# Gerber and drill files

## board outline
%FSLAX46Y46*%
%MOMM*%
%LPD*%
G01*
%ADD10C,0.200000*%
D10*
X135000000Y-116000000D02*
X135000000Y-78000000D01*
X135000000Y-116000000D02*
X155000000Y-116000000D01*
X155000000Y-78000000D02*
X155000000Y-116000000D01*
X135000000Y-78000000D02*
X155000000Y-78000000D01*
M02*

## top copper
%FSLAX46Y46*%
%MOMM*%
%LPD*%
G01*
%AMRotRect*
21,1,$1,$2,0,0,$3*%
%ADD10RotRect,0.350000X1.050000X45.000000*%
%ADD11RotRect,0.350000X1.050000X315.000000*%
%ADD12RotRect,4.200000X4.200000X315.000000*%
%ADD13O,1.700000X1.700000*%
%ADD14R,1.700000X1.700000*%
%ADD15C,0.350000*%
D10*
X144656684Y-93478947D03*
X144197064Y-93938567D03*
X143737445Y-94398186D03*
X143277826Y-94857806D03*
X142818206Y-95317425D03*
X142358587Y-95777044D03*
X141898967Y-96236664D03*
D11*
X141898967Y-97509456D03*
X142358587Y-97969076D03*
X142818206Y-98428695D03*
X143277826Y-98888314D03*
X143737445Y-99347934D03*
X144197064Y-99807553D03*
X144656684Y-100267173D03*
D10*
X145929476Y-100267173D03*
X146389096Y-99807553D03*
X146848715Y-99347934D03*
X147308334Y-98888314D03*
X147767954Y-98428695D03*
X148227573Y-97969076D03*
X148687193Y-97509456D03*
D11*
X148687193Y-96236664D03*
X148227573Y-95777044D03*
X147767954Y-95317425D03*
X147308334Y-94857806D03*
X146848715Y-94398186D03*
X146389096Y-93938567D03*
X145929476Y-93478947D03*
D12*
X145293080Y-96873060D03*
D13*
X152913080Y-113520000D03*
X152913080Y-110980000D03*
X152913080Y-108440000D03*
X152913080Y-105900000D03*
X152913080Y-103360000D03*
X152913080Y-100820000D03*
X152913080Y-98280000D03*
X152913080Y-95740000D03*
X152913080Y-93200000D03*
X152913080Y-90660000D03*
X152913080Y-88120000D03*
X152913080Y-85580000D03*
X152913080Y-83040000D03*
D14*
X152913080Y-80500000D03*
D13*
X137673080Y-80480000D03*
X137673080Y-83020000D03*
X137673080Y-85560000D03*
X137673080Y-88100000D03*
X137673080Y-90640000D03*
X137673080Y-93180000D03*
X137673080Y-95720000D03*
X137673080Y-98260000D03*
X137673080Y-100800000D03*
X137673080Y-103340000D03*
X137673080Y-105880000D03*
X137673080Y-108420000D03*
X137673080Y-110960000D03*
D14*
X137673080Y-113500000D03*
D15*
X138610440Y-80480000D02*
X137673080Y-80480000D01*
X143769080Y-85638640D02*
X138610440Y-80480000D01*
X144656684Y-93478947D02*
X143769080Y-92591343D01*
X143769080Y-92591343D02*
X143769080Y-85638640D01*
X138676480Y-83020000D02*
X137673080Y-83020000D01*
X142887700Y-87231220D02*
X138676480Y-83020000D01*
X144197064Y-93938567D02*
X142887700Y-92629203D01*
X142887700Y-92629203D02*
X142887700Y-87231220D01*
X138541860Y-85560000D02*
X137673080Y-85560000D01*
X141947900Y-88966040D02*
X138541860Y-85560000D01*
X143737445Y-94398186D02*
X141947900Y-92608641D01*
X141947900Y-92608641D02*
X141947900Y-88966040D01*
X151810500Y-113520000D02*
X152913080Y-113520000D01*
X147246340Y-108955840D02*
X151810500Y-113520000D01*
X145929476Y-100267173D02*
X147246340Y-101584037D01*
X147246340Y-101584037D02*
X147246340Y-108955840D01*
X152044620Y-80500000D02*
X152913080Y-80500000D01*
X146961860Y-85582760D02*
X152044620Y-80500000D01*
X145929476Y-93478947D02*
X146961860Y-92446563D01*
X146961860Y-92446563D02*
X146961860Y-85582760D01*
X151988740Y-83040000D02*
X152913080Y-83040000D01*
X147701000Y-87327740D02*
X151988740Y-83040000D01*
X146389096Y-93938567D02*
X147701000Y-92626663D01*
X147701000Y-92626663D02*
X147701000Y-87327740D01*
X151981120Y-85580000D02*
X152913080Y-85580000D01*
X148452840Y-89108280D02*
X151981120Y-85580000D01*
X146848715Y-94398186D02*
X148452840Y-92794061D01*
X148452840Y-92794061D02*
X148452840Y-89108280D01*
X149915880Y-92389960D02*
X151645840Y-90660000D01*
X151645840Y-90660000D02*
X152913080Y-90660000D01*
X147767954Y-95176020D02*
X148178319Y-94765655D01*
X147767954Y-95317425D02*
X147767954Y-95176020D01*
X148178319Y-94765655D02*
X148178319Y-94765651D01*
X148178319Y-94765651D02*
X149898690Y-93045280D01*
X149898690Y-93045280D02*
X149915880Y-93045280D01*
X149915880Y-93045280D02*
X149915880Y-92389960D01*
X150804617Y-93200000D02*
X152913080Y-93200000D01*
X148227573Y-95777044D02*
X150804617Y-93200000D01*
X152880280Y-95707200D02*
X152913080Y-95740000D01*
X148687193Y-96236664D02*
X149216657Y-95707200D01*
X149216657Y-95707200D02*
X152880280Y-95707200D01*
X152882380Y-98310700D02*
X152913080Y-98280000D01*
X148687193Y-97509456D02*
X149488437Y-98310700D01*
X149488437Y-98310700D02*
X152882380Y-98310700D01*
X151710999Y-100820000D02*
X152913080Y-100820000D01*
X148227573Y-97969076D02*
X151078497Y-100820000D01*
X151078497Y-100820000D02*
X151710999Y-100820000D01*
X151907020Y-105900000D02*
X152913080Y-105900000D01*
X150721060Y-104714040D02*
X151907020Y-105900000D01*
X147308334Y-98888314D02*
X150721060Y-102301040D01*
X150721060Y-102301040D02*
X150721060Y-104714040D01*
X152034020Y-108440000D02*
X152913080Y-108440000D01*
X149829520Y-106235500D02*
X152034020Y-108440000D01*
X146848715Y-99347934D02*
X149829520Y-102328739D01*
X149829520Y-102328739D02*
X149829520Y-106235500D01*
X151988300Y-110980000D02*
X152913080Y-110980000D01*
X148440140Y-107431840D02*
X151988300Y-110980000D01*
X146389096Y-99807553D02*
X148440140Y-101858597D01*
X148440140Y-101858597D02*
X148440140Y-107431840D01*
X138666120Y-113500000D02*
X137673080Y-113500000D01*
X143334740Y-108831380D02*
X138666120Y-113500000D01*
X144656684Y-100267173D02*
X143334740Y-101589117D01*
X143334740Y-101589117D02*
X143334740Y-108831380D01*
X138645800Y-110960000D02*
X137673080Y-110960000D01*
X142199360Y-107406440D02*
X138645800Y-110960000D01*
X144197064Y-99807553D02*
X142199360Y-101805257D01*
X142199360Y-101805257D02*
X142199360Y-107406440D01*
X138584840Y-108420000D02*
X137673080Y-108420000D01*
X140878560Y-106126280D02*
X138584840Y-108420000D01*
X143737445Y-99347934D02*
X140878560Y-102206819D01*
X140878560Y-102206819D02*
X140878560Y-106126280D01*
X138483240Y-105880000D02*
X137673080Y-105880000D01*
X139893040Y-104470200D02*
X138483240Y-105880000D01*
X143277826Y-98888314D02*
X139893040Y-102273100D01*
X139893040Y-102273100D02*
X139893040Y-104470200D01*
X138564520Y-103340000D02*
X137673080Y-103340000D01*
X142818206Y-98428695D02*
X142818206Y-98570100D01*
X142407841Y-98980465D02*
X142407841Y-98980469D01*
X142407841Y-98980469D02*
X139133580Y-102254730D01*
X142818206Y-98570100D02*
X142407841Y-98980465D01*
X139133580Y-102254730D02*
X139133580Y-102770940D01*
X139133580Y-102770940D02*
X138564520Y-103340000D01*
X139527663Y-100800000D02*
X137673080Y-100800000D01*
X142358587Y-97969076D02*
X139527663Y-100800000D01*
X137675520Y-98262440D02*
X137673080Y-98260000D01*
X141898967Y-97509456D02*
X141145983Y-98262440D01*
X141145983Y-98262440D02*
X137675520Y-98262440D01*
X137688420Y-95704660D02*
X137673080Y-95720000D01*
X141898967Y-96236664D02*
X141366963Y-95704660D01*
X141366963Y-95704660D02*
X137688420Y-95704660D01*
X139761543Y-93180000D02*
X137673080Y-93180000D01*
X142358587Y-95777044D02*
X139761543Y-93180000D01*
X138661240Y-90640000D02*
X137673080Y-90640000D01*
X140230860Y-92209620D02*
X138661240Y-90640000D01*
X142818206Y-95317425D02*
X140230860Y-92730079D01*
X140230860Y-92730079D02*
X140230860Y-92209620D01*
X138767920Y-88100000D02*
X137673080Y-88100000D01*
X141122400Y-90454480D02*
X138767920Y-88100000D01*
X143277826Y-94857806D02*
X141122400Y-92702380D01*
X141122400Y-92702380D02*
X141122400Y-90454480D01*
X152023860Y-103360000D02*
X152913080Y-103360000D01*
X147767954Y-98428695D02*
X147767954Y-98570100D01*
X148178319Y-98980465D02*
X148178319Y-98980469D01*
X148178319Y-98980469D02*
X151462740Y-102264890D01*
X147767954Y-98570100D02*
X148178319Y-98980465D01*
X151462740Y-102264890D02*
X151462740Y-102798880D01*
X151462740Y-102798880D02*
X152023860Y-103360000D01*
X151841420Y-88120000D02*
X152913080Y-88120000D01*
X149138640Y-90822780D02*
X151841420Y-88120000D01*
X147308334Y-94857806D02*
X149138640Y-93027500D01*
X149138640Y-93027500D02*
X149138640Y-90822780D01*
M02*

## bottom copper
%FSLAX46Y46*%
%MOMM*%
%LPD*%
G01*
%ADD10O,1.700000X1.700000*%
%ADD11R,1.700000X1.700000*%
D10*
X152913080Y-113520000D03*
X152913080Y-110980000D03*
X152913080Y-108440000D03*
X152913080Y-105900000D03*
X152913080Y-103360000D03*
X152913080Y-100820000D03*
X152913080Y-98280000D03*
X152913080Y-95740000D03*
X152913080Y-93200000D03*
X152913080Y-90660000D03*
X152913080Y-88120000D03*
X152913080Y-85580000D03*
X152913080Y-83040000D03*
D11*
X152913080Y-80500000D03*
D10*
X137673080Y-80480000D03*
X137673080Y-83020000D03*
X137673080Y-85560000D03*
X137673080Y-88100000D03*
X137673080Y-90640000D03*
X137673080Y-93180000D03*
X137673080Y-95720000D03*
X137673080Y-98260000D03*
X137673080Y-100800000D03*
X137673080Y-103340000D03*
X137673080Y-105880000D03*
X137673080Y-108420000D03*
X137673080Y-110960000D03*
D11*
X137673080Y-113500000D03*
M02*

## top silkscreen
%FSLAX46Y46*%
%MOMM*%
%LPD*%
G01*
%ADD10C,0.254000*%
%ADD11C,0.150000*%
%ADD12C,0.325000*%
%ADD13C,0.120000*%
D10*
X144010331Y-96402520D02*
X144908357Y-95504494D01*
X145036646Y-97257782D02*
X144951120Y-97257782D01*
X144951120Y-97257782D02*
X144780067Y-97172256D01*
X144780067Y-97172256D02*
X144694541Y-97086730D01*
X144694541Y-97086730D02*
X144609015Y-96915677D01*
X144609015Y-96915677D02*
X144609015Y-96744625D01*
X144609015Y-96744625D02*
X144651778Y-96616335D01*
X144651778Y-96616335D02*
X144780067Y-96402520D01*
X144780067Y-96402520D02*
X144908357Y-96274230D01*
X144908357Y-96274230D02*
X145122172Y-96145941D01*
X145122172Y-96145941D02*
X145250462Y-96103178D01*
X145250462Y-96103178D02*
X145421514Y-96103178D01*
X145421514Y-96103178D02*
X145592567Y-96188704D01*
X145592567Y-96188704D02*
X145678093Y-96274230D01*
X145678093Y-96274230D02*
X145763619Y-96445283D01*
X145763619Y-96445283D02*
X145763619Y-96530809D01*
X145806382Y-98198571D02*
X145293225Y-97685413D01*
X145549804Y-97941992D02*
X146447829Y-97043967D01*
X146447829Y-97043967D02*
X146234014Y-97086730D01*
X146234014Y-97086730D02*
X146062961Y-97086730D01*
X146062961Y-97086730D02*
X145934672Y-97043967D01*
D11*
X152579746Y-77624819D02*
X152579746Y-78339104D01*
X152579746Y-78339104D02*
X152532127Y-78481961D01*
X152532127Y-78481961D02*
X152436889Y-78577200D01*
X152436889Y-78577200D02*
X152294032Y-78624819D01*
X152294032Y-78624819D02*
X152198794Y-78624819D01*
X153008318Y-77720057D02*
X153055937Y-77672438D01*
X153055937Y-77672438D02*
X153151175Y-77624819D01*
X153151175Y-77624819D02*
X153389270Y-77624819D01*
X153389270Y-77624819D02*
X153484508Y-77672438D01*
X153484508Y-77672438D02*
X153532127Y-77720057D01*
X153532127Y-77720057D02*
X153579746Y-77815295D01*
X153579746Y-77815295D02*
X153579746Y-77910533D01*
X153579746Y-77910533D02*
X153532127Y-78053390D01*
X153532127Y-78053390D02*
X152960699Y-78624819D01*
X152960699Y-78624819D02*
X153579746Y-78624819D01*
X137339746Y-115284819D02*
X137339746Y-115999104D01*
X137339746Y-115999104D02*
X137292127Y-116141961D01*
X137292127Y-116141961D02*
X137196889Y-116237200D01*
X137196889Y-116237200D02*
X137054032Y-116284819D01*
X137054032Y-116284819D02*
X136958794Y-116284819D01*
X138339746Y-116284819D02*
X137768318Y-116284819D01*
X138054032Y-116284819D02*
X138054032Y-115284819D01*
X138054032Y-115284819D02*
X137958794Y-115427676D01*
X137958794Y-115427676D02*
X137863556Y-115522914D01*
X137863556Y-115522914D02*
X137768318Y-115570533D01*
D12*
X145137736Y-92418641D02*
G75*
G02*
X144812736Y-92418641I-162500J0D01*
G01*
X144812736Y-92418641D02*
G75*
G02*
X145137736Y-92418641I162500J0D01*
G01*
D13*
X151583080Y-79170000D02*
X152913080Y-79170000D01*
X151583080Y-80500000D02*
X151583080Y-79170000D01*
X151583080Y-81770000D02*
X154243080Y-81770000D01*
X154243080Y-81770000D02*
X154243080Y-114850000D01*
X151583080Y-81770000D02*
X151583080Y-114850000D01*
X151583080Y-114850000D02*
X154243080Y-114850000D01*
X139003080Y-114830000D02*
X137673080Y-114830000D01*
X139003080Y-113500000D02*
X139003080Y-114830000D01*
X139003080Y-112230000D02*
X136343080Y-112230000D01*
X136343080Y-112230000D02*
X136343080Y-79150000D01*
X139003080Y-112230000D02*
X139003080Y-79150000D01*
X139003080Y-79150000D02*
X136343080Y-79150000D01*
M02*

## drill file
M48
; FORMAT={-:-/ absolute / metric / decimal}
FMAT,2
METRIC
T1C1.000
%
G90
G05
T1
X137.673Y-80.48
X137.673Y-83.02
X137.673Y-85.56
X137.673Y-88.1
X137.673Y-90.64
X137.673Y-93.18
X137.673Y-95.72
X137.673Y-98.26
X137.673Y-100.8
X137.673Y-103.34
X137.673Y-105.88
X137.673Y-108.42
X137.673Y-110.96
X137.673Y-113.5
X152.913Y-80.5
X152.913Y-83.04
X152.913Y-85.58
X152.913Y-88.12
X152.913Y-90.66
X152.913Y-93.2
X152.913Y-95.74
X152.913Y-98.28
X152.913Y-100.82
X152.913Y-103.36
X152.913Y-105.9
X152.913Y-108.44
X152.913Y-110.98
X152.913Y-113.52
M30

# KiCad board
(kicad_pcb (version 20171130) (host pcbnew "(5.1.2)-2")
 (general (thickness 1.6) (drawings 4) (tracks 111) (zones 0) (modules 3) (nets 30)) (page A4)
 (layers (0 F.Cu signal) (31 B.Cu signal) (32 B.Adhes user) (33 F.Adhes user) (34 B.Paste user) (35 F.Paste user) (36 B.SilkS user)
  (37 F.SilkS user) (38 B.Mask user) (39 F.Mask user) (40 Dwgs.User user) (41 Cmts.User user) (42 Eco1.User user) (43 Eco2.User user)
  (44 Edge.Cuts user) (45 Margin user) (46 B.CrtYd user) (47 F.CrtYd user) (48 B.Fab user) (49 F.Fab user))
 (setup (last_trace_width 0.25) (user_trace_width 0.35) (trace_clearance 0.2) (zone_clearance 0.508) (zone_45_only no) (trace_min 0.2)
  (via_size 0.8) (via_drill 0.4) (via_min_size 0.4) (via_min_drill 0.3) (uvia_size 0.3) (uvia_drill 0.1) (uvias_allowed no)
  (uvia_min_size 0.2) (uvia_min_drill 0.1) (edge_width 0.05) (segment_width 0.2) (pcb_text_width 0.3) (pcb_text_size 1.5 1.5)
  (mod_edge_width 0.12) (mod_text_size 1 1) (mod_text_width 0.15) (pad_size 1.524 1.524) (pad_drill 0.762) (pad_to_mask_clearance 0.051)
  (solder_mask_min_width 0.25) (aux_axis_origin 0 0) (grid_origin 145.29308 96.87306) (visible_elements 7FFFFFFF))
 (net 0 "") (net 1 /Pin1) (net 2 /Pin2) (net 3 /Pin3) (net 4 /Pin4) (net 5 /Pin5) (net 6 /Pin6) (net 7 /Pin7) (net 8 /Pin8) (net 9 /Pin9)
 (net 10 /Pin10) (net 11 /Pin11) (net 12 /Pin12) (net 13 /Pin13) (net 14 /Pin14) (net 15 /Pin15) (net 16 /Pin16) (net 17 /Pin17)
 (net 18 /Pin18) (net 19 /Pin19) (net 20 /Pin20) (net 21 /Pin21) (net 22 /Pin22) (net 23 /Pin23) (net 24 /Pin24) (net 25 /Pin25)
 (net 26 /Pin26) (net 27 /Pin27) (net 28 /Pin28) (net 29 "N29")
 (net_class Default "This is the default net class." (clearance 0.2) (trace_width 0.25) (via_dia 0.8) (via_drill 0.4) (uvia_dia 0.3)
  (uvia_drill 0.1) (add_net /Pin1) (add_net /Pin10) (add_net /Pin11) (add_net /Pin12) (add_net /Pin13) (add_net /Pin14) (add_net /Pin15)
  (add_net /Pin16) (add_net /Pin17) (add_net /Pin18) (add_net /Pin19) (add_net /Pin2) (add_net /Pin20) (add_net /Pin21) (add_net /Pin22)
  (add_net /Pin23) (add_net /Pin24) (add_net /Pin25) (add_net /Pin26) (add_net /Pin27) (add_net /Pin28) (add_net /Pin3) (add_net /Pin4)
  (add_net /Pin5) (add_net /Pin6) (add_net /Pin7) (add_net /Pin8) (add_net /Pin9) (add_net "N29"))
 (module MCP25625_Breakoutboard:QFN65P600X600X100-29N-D (layer F.Cu) (at 145.29308 96.87306 315)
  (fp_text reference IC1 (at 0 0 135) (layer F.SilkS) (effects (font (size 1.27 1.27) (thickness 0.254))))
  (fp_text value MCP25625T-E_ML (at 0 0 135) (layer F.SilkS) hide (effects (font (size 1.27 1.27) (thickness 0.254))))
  (fp_circle (center -3.3745 -2.925) (end -3.3745 -2.7625) (layer F.SilkS) (width 0.325))
  (pad 1 smd rect (at -2.85 -1.95 45) (size 0.35 1.05) (layers F.Cu F.Paste F.Mask) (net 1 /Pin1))
  (pad 2 smd rect (at -2.85 -1.3 45) (size 0.35 1.05) (layers F.Cu F.Paste F.Mask) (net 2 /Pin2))
  (pad 3 smd rect (at -2.85 -0.65 45) (size 0.35 1.05) (layers F.Cu F.Paste F.Mask) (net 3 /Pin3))
  (pad 4 smd rect (at -2.85 0 45) (size 0.35 1.05) (layers F.Cu F.Paste F.Mask) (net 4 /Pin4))
  (pad 5 smd rect (at -2.85 0.65 45) (size 0.35 1.05) (layers F.Cu F.Paste F.Mask) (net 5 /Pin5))
  (pad 6 smd rect (at -2.85 1.3 45) (size 0.35 1.05) (layers F.Cu F.Paste F.Mask) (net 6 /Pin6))
  (pad 7 smd rect (at -2.85 1.95 45) (size 0.35 1.05) (layers F.Cu F.Paste F.Mask) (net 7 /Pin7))
  (pad 8 smd rect (at -1.95 2.85 315) (size 0.35 1.05) (layers F.Cu F.Paste F.Mask) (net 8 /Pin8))
  (pad 9 smd rect (at -1.3 2.85 315) (size 0.35 1.05) (layers F.Cu F.Paste F.Mask) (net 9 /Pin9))
  (pad 10 smd rect (at -0.65 2.85 315) (size 0.35 1.05) (layers F.Cu F.Paste F.Mask) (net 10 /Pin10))
  (pad 11 smd rect (at 0 2.85 315) (size 0.35 1.05) (layers F.Cu F.Paste F.Mask) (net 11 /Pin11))
  (pad 12 smd rect (at 0.65 2.85 315) (size 0.35 1.05) (layers F.Cu F.Paste F.Mask) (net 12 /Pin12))
  (pad 13 smd rect (at 1.3 2.85 315) (size 0.35 1.05) (layers F.Cu F.Paste F.Mask) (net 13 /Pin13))
  (pad 14 smd rect (at 1.95 2.85 315) (size 0.35 1.05) (layers F.Cu F.Paste F.Mask) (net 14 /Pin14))
  (pad 15 smd rect (at 2.85 1.95 45) (size 0.35 1.05) (layers F.Cu F.Paste F.Mask) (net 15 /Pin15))
  (pad 16 smd rect (at 2.85 1.3 45) (size 0.35 1.05) (layers F.Cu F.Paste F.Mask) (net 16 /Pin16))
  (pad 17 smd rect (at 2.85 0.65 45) (size 0.35 1.05) (layers F.Cu F.Paste F.Mask) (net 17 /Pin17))
  (pad 18 smd rect (at 2.85 0 45) (size 0.35 1.05) (layers F.Cu F.Paste F.Mask) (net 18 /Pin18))
  (pad 19 smd rect (at 2.85 -0.65 45) (size 0.35 1.05) (layers F.Cu F.Paste F.Mask) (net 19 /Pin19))
  (pad 20 smd rect (at 2.85 -1.3 45) (size 0.35 1.05) (layers F.Cu F.Paste F.Mask) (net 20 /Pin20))
  (pad 21 smd rect (at 2.85 -1.95 45) (size 0.35 1.05) (layers F.Cu F.Paste F.Mask) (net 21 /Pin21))
  (pad 22 smd rect (at 1.95 -2.85 315) (size 0.35 1.05) (layers F.Cu F.Paste F.Mask) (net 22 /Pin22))
  (pad 23 smd rect (at 1.3 -2.85 315) (size 0.35 1.05) (layers F.Cu F.Paste F.Mask) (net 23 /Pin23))
  (pad 24 smd rect (at 0.65 -2.85 315) (size 0.35 1.05) (layers F.Cu F.Paste F.Mask) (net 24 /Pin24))
  (pad 25 smd rect (at 0 -2.85 315) (size 0.35 1.05) (layers F.Cu F.Paste F.Mask) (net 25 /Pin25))
  (pad 26 smd rect (at -0.65 -2.85 315) (size 0.35 1.05) (layers F.Cu F.Paste F.Mask) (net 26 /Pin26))
  (pad 27 smd rect (at -1.3 -2.85 315) (size 0.35 1.05) (layers F.Cu F.Paste F.Mask) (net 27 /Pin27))
  (pad 28 smd rect (at -1.95 -2.85 315) (size 0.35 1.05) (layers F.Cu F.Paste F.Mask) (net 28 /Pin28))
  (pad 29 smd rect (at 0 0 315) (size 4.2 4.2) (layers F.Cu F.Paste F.Mask) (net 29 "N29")))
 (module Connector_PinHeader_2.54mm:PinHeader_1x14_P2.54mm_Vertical (layer F.Cu) (at 152.91308 80.5)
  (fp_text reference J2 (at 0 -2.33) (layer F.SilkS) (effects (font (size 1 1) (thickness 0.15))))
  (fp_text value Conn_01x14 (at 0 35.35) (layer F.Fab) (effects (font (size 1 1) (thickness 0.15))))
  (fp_line (start -1.33 -1.33) (end 0 -1.33) (layer F.SilkS) (width 0.12))
  (fp_line (start -1.33 0) (end -1.33 -1.33) (layer F.SilkS) (width 0.12))
  (fp_line (start -1.33 1.27) (end 1.33 1.27) (layer F.SilkS) (width 0.12))
  (fp_line (start 1.33 1.27) (end 1.33 34.35) (layer F.SilkS) (width 0.12))
  (fp_line (start -1.33 1.27) (end -1.33 34.35) (layer F.SilkS) (width 0.12))
  (fp_line (start -1.33 34.35) (end 1.33 34.35) (layer F.SilkS) (width 0.12))
  (pad 14 thru_hole oval (at 0 33.02) (size 1.7 1.7) (drill 1) (layers *.Cu *.Mask) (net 15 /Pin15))
  (pad 13 thru_hole oval (at 0 30.48) (size 1.7 1.7) (drill 1) (layers *.Cu *.Mask) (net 16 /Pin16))
  (pad 12 thru_hole oval (at 0 27.94) (size 1.7 1.7) (drill 1) (layers *.Cu *.Mask) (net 17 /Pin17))
  (pad 11 thru_hole oval (at 0 25.4) (size 1.7 1.7) (drill 1) (layers *.Cu *.Mask) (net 18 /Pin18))
  (pad 10 thru_hole oval (at 0 22.86) (size 1.7 1.7) (drill 1) (layers *.Cu *.Mask) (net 19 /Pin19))
  (pad 9 thru_hole oval (at 0 20.32) (size 1.7 1.7) (drill 1) (layers *.Cu *.Mask) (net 20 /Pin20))
  (pad 8 thru_hole oval (at 0 17.78) (size 1.7 1.7) (drill 1) (layers *.Cu *.Mask) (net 21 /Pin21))
  (pad 7 thru_hole oval (at 0 15.24) (size 1.7 1.7) (drill 1) (layers *.Cu *.Mask) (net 22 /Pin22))
  (pad 6 thru_hole oval (at 0 12.7) (size 1.7 1.7) (drill 1) (layers *.Cu *.Mask) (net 23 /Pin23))
  (pad 5 thru_hole oval (at 0 10.16) (size 1.7 1.7) (drill 1) (layers *.Cu *.Mask) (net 24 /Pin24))
  (pad 4 thru_hole oval (at 0 7.62) (size 1.7 1.7) (drill 1) (layers *.Cu *.Mask) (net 25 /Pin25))
  (pad 3 thru_hole oval (at 0 5.08) (size 1.7 1.7) (drill 1) (layers *.Cu *.Mask) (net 26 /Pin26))
  (pad 2 thru_hole oval (at 0 2.54) (size 1.7 1.7) (drill 1) (layers *.Cu *.Mask) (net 27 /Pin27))
  (pad 1 thru_hole rect (at 0 0) (size 1.7 1.7) (drill 1) (layers *.Cu *.Mask) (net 28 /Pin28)))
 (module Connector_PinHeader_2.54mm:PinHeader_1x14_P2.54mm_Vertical (layer F.Cu) (at 137.67308 113.5 180)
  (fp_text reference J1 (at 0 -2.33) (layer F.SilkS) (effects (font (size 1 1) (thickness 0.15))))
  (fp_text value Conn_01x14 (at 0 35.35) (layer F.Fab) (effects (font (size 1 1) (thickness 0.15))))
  (fp_line (start -1.33 -1.33) (end 0 -1.33) (layer F.SilkS) (width 0.12))
  (fp_line (start -1.33 0) (end -1.33 -1.33) (layer F.SilkS) (width 0.12))
  (fp_line (start -1.33 1.27) (end 1.33 1.27) (layer F.SilkS) (width 0.12))
  (fp_line (start 1.33 1.27) (end 1.33 34.35) (layer F.SilkS) (width 0.12))
  (fp_line (start -1.33 1.27) (end -1.33 34.35) (layer F.SilkS) (width 0.12))
  (fp_line (start -1.33 34.35) (end 1.33 34.35) (layer F.SilkS) (width 0.12))
  (pad 14 thru_hole oval (at 0 33.02 180) (size 1.7 1.7) (drill 1) (layers *.Cu *.Mask) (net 1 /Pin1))
  (pad 13 thru_hole oval (at 0 30.48 180) (size 1.7 1.7) (drill 1) (layers *.Cu *.Mask) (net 2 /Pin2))
  (pad 12 thru_hole oval (at 0 27.94 180) (size 1.7 1.7) (drill 1) (layers *.Cu *.Mask) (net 3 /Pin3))
  (pad 11 thru_hole oval (at 0 25.4 180) (size 1.7 1.7) (drill 1) (layers *.Cu *.Mask) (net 4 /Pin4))
  (pad 10 thru_hole oval (at 0 22.86 180) (size 1.7 1.7) (drill 1) (layers *.Cu *.Mask) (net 5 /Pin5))
  (pad 9 thru_hole oval (at 0 20.32 180) (size 1.7 1.7) (drill 1) (layers *.Cu *.Mask) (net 6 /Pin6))
  (pad 8 thru_hole oval (at 0 17.78 180) (size 1.7 1.7) (drill 1) (layers *.Cu *.Mask) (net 7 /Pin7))
  (pad 7 thru_hole oval (at 0 15.24 180) (size 1.7 1.7) (drill 1) (layers *.Cu *.Mask) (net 8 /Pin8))
  (pad 6 thru_hole oval (at 0 12.7 180) (size 1.7 1.7) (drill 1) (layers *.Cu *.Mask) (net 9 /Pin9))
  (pad 5 thru_hole oval (at 0 10.16 180) (size 1.7 1.7) (drill 1) (layers *.Cu *.Mask) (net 10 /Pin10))
  (pad 4 thru_hole oval (at 0 7.62 180) (size 1.7 1.7) (drill 1) (layers *.Cu *.Mask) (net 11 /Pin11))
  (pad 3 thru_hole oval (at 0 5.08 180) (size 1.7 1.7) (drill 1) (layers *.Cu *.Mask) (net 12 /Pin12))
  (pad 2 thru_hole oval (at 0 2.54 180) (size 1.7 1.7) (drill 1) (layers *.Cu *.Mask) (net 13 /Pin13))
  (pad 1 thru_hole rect (at 0 0 180) (size 1.7 1.7) (drill 1) (layers *.Cu *.Mask) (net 14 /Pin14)))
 (gr_line (start 135 116) (end 135 78) (layer Edge.Cuts) (width 0.2))
 (gr_line (start 135 116) (end 155 116) (layer Edge.Cuts) (width 0.2))
 (gr_line (start 155 78) (end 155 116) (layer Edge.Cuts) (width 0.2))
 (gr_line (start 135 78) (end 155 78) (layer Edge.Cuts) (width 0.2))
 (segment (start 138.61044 80.48) (end 137.67308 80.48) (width 0.35) (layer F.Cu) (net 1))
 (segment (start 143.76908 85.63864) (end 138.61044 80.48) (width 0.35) (layer F.Cu) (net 1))
 (segment (start 144.656684 93.478947) (end 143.76908 92.591343) (width 0.35) (layer F.Cu) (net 1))
 (segment (start 143.76908 92.591343) (end 143.76908 85.63864) (width 0.35) (layer F.Cu) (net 1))
 (segment (start 138.67648 83.02) (end 137.67308 83.02) (width 0.35) (layer F.Cu) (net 2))
 (segment (start 142.8877 87.23122) (end 138.67648 83.02) (width 0.35) (layer F.Cu) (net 2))
 (segment (start 144.197064 93.938567) (end 142.8877 92.629203) (width 0.35) (layer F.Cu) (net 2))
 (segment (start 142.8877 92.629203) (end 142.8877 87.23122) (width 0.35) (layer F.Cu) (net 2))
 (segment (start 138.54186 85.56) (end 137.67308 85.56) (width 0.35) (layer F.Cu) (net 3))
 (segment (start 141.9479 88.96604) (end 138.54186 85.56) (width 0.35) (layer F.Cu) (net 3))
 (segment (start 143.737445 94.398186) (end 141.9479 92.608641) (width 0.35) (layer F.Cu) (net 3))
 (segment (start 141.9479 92.608641) (end 141.9479 88.96604) (width 0.35) (layer F.Cu) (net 3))
 (segment (start 151.8105 113.52) (end 152.91308 113.52) (width 0.35) (layer F.Cu) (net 15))
 (segment (start 147.24634 108.95584) (end 151.8105 113.52) (width 0.35) (layer F.Cu) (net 15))
 (segment (start 145.929476 100.267173) (end 147.24634 101.584037) (width 0.35) (layer F.Cu) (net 15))
 (segment (start 147.24634 101.584037) (end 147.24634 108.95584) (width 0.35) (layer F.Cu) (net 15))
 (segment (start 152.04462 80.5) (end 152.91308 80.5) (width 0.35) (layer F.Cu) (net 28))
 (segment (start 146.96186 85.58276) (end 152.04462 80.5) (width 0.35) (layer F.Cu) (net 28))
 (segment (start 145.929476 93.478947) (end 146.96186 92.446563) (width 0.35) (layer F.Cu) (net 28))
 (segment (start 146.96186 92.446563) (end 146.96186 85.58276) (width 0.35) (layer F.Cu) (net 28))
 (segment (start 151.98874 83.04) (end 152.91308 83.04) (width 0.35) (layer F.Cu) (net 27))
 (segment (start 147.701 87.32774) (end 151.98874 83.04) (width 0.35) (layer F.Cu) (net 27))
 (segment (start 146.389096 93.938567) (end 147.701 92.626663) (width 0.35) (layer F.Cu) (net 27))
 (segment (start 147.701 92.626663) (end 147.701 87.32774) (width 0.35) (layer F.Cu) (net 27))
 (segment (start 151.98112 85.58) (end 152.91308 85.58) (width 0.35) (layer F.Cu) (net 26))
 (segment (start 148.45284 89.10828) (end 151.98112 85.58) (width 0.35) (layer F.Cu) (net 26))
 (segment (start 146.848715 94.398186) (end 148.45284 92.794061) (width 0.35) (layer F.Cu) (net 26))
 (segment (start 148.45284 92.794061) (end 148.45284 89.10828) (width 0.35) (layer F.Cu) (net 26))
 (segment (start 149.91588 92.38996) (end 151.64584 90.66) (width 0.35) (layer F.Cu) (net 24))
 (segment (start 151.64584 90.66) (end 152.91308 90.66) (width 0.35) (layer F.Cu) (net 24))
 (segment (start 147.767954 95.17602) (end 148.178319 94.765655) (width 0.35) (layer F.Cu) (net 24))
 (segment (start 147.767954 95.317425) (end 147.767954 95.17602) (width 0.35) (layer F.Cu) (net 24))
 (segment (start 148.178319 94.765655) (end 148.178319 94.765651) (width 0.35) (layer F.Cu) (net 24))
 (segment (start 148.178319 94.765651) (end 149.89869 93.04528) (width 0.35) (layer F.Cu) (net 24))
 (segment (start 149.89869 93.04528) (end 149.91588 93.04528) (width 0.35) (layer F.Cu) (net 24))
 (segment (start 149.91588 93.04528) (end 149.91588 92.38996) (width 0.35) (layer F.Cu) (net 24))
 (segment (start 150.804617 93.2) (end 152.91308 93.2) (width 0.35) (layer F.Cu) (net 23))
 (segment (start 148.227573 95.777044) (end 150.804617 93.2) (width 0.35) (layer F.Cu) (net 23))
 (segment (start 152.88028 95.7072) (end 152.91308 95.74) (width 0.35) (layer F.Cu) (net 22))
 (segment (start 148.687193 96.236664) (end 149.216657 95.7072) (width 0.35) (layer F.Cu) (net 22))
 (segment (start 149.216657 95.7072) (end 152.88028 95.7072) (width 0.35) (layer F.Cu) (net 22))
 (segment (start 152.88238 98.3107) (end 152.91308 98.28) (width 0.35) (layer F.Cu) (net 21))
 (segment (start 148.687193 97.509456) (end 149.488437 98.3107) (width 0.35) (layer F.Cu) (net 21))
 (segment (start 149.488437 98.3107) (end 152.88238 98.3107) (width 0.35) (layer F.Cu) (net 21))
 (segment (start 151.710999 100.82) (end 152.91308 100.82) (width 0.35) (layer F.Cu) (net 20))
 (segment (start 148.227573 97.969076) (end 151.078497 100.82) (width 0.35) (layer F.Cu) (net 20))
 (segment (start 151.078497 100.82) (end 151.710999 100.82) (width 0.35) (layer F.Cu) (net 20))
 (segment (start 151.90702 105.9) (end 152.91308 105.9) (width 0.35) (layer F.Cu) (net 18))
 (segment (start 150.72106 104.71404) (end 151.90702 105.9) (width 0.35) (layer F.Cu) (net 18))
 (segment (start 147.308334 98.888314) (end 150.72106 102.30104) (width 0.35) (layer F.Cu) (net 18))
 (segment (start 150.72106 102.30104) (end 150.72106 104.71404) (width 0.35) (layer F.Cu) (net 18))
 (segment (start 152.03402 108.44) (end 152.91308 108.44) (width 0.35) (layer F.Cu) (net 17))
 (segment (start 149.82952 106.2355) (end 152.03402 108.44) (width 0.35) (layer F.Cu) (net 17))
 (segment (start 146.848715 99.347934) (end 149.82952 102.328739) (width 0.35) (layer F.Cu) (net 17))
 (segment (start 149.82952 102.328739) (end 149.82952 106.2355) (width 0.35) (layer F.Cu) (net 17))
 (segment (start 151.9883 110.98) (end 152.91308 110.98) (width 0.35) (layer F.Cu) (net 16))
 (segment (start 148.44014 107.43184) (end 151.9883 110.98) (width 0.35) (layer F.Cu) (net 16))
 (segment (start 146.389096 99.807553) (end 148.44014 101.858597) (width 0.35) (layer F.Cu) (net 16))
 (segment (start 148.44014 101.858597) (end 148.44014 107.43184) (width 0.35) (layer F.Cu) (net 16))
 (segment (start 138.66612 113.5) (end 137.67308 113.5) (width 0.35) (layer F.Cu) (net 14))
 (segment (start 143.33474 108.83138) (end 138.66612 113.5) (width 0.35) (layer F.Cu) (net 14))
 (segment (start 144.656684 100.267173) (end 143.33474 101.589117) (width 0.35) (layer F.Cu) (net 14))
 (segment (start 143.33474 101.589117) (end 143.33474 108.83138) (width 0.35) (layer F.Cu) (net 14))
 (segment (start 138.6458 110.96) (end 137.67308 110.96) (width 0.35) (layer F.Cu) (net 13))
 (segment (start 142.19936 107.40644) (end 138.6458 110.96) (width 0.35) (layer F.Cu) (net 13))
 (segment (start 144.197064 99.807553) (end 142.19936 101.805257) (width 0.35) (layer F.Cu) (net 13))
 (segment (start 142.19936 101.805257) (end 142.19936 107.40644) (width 0.35) (layer F.Cu) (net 13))
 (segment (start 138.58484 108.42) (end 137.67308 108.42) (width 0.35) (layer F.Cu) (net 12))
 (segment (start 140.87856 106.12628) (end 138.58484 108.42) (width 0.35) (layer F.Cu) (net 12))
 (segment (start 143.737445 99.347934) (end 140.87856 102.206819) (width 0.35) (layer F.Cu) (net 12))
 (segment (start 140.87856 102.206819) (end 140.87856 106.12628) (width 0.35) (layer F.Cu) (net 12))
 (segment (start 138.48324 105.88) (end 137.67308 105.88) (width 0.35) (layer F.Cu) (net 11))
 (segment (start 139.89304 104.4702) (end 138.48324 105.88) (width 0.35) (layer F.Cu) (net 11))
 (segment (start 143.277826 98.888314) (end 139.89304 102.2731) (width 0.35) (layer F.Cu) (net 11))
 (segment (start 139.89304 102.2731) (end 139.89304 104.4702) (width 0.35) (layer F.Cu) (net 11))
 (segment (start 138.56452 103.34) (end 137.67308 103.34) (width 0.35) (layer F.Cu) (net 10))
 (segment (start 142.818206 98.428695) (end 142.818206 98.5701) (width 0.35) (layer F.Cu) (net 10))
 (segment (start 142.407841 98.980465) (end 142.407841 98.980469) (width 0.35) (layer F.Cu) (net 10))
 (segment (start 142.407841 98.980469) (end 139.13358 102.25473) (width 0.35) (layer F.Cu) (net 10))
 (segment (start 142.818206 98.5701) (end 142.407841 98.980465) (width 0.35) (layer F.Cu) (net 10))
 (segment (start 139.13358 102.25473) (end 139.13358 102.77094) (width 0.35) (layer F.Cu) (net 10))
 (segment (start 139.13358 102.77094) (end 138.56452 103.34) (width 0.35) (layer F.Cu) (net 10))
 (segment (start 139.527663 100.8) (end 137.67308 100.8) (width 0.35) (layer F.Cu) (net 9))
 (segment (start 142.358587 97.969076) (end 139.527663 100.8) (width 0.35) (layer F.Cu) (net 9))
 (segment (start 137.67552 98.26244) (end 137.67308 98.26) (width 0.35) (layer F.Cu) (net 8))
 (segment (start 141.898967 97.509456) (end 141.145983 98.26244) (width 0.35) (layer F.Cu) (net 8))
 (segment (start 141.145983 98.26244) (end 137.67552 98.26244) (width 0.35) (layer F.Cu) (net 8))
 (segment (start 137.68842 95.70466) (end 137.67308 95.72) (width 0.35) (layer F.Cu) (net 7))
 (segment (start 141.898967 96.236664) (end 141.366963 95.70466) (width 0.35) (layer F.Cu) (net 7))
 (segment (start 141.366963 95.70466) (end 137.68842 95.70466) (width 0.35) (layer F.Cu) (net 7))
 (segment (start 139.761543 93.18) (end 137.67308 93.18) (width 0.35) (layer F.Cu) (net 6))
 (segment (start 142.358587 95.777044) (end 139.761543 93.18) (width 0.35) (layer F.Cu) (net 6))
 (segment (start 138.66124 90.64) (end 137.67308 90.64) (width 0.35) (layer F.Cu) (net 5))
 (segment (start 140.23086 92.20962) (end 138.66124 90.64) (width 0.35) (layer F.Cu) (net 5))
 (segment (start 142.818206 95.317425) (end 140.23086 92.730079) (width 0.35) (layer F.Cu) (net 5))
 (segment (start 140.23086 92.730079) (end 140.23086 92.20962) (width 0.35) (layer F.Cu) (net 5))
 (segment (start 138.76792 88.1) (end 137.67308 88.1) (width 0.35) (layer F.Cu) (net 4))
 (segment (start 141.1224 90.45448) (end 138.76792 88.1) (width 0.35) (layer F.Cu) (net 4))
 (segment (start 143.277826 94.857806) (end 141.1224 92.70238) (width 0.35) (layer F.Cu) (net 4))
 (segment (start 141.1224 92.70238) (end 141.1224 90.45448) (width 0.35) (layer F.Cu) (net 4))
 (segment (start 152.02386 103.36) (end 152.91308 103.36) (width 0.35) (layer F.Cu) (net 19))
 (segment (start 147.767954 98.428695) (end 147.767954 98.5701) (width 0.35) (layer F.Cu) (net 19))
 (segment (start 148.178319 98.980465) (end 148.178319 98.980469) (width 0.35) (layer F.Cu) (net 19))
 (segment (start 148.178319 98.980469) (end 151.46274 102.26489) (width 0.35) (layer F.Cu) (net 19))
 (segment (start 147.767954 98.5701) (end 148.178319 98.980465) (width 0.35) (layer F.Cu) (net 19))
 (segment (start 151.46274 102.26489) (end 151.46274 102.79888) (width 0.35) (layer F.Cu) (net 19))
 (segment (start 151.46274 102.79888) (end 152.02386 103.36) (width 0.35) (layer F.Cu) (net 19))
 (segment (start 151.84142 88.12) (end 152.91308 88.12) (width 0.35) (layer F.Cu) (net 25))
 (segment (start 149.13864 90.82278) (end 151.84142 88.12) (width 0.35) (layer F.Cu) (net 25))
 (segment (start 147.308334 94.857806) (end 149.13864 93.0275) (width 0.35) (layer F.Cu) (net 25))
 (segment (start 149.13864 93.0275) (end 149.13864 90.82278) (width 0.35) (layer F.Cu) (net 25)))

